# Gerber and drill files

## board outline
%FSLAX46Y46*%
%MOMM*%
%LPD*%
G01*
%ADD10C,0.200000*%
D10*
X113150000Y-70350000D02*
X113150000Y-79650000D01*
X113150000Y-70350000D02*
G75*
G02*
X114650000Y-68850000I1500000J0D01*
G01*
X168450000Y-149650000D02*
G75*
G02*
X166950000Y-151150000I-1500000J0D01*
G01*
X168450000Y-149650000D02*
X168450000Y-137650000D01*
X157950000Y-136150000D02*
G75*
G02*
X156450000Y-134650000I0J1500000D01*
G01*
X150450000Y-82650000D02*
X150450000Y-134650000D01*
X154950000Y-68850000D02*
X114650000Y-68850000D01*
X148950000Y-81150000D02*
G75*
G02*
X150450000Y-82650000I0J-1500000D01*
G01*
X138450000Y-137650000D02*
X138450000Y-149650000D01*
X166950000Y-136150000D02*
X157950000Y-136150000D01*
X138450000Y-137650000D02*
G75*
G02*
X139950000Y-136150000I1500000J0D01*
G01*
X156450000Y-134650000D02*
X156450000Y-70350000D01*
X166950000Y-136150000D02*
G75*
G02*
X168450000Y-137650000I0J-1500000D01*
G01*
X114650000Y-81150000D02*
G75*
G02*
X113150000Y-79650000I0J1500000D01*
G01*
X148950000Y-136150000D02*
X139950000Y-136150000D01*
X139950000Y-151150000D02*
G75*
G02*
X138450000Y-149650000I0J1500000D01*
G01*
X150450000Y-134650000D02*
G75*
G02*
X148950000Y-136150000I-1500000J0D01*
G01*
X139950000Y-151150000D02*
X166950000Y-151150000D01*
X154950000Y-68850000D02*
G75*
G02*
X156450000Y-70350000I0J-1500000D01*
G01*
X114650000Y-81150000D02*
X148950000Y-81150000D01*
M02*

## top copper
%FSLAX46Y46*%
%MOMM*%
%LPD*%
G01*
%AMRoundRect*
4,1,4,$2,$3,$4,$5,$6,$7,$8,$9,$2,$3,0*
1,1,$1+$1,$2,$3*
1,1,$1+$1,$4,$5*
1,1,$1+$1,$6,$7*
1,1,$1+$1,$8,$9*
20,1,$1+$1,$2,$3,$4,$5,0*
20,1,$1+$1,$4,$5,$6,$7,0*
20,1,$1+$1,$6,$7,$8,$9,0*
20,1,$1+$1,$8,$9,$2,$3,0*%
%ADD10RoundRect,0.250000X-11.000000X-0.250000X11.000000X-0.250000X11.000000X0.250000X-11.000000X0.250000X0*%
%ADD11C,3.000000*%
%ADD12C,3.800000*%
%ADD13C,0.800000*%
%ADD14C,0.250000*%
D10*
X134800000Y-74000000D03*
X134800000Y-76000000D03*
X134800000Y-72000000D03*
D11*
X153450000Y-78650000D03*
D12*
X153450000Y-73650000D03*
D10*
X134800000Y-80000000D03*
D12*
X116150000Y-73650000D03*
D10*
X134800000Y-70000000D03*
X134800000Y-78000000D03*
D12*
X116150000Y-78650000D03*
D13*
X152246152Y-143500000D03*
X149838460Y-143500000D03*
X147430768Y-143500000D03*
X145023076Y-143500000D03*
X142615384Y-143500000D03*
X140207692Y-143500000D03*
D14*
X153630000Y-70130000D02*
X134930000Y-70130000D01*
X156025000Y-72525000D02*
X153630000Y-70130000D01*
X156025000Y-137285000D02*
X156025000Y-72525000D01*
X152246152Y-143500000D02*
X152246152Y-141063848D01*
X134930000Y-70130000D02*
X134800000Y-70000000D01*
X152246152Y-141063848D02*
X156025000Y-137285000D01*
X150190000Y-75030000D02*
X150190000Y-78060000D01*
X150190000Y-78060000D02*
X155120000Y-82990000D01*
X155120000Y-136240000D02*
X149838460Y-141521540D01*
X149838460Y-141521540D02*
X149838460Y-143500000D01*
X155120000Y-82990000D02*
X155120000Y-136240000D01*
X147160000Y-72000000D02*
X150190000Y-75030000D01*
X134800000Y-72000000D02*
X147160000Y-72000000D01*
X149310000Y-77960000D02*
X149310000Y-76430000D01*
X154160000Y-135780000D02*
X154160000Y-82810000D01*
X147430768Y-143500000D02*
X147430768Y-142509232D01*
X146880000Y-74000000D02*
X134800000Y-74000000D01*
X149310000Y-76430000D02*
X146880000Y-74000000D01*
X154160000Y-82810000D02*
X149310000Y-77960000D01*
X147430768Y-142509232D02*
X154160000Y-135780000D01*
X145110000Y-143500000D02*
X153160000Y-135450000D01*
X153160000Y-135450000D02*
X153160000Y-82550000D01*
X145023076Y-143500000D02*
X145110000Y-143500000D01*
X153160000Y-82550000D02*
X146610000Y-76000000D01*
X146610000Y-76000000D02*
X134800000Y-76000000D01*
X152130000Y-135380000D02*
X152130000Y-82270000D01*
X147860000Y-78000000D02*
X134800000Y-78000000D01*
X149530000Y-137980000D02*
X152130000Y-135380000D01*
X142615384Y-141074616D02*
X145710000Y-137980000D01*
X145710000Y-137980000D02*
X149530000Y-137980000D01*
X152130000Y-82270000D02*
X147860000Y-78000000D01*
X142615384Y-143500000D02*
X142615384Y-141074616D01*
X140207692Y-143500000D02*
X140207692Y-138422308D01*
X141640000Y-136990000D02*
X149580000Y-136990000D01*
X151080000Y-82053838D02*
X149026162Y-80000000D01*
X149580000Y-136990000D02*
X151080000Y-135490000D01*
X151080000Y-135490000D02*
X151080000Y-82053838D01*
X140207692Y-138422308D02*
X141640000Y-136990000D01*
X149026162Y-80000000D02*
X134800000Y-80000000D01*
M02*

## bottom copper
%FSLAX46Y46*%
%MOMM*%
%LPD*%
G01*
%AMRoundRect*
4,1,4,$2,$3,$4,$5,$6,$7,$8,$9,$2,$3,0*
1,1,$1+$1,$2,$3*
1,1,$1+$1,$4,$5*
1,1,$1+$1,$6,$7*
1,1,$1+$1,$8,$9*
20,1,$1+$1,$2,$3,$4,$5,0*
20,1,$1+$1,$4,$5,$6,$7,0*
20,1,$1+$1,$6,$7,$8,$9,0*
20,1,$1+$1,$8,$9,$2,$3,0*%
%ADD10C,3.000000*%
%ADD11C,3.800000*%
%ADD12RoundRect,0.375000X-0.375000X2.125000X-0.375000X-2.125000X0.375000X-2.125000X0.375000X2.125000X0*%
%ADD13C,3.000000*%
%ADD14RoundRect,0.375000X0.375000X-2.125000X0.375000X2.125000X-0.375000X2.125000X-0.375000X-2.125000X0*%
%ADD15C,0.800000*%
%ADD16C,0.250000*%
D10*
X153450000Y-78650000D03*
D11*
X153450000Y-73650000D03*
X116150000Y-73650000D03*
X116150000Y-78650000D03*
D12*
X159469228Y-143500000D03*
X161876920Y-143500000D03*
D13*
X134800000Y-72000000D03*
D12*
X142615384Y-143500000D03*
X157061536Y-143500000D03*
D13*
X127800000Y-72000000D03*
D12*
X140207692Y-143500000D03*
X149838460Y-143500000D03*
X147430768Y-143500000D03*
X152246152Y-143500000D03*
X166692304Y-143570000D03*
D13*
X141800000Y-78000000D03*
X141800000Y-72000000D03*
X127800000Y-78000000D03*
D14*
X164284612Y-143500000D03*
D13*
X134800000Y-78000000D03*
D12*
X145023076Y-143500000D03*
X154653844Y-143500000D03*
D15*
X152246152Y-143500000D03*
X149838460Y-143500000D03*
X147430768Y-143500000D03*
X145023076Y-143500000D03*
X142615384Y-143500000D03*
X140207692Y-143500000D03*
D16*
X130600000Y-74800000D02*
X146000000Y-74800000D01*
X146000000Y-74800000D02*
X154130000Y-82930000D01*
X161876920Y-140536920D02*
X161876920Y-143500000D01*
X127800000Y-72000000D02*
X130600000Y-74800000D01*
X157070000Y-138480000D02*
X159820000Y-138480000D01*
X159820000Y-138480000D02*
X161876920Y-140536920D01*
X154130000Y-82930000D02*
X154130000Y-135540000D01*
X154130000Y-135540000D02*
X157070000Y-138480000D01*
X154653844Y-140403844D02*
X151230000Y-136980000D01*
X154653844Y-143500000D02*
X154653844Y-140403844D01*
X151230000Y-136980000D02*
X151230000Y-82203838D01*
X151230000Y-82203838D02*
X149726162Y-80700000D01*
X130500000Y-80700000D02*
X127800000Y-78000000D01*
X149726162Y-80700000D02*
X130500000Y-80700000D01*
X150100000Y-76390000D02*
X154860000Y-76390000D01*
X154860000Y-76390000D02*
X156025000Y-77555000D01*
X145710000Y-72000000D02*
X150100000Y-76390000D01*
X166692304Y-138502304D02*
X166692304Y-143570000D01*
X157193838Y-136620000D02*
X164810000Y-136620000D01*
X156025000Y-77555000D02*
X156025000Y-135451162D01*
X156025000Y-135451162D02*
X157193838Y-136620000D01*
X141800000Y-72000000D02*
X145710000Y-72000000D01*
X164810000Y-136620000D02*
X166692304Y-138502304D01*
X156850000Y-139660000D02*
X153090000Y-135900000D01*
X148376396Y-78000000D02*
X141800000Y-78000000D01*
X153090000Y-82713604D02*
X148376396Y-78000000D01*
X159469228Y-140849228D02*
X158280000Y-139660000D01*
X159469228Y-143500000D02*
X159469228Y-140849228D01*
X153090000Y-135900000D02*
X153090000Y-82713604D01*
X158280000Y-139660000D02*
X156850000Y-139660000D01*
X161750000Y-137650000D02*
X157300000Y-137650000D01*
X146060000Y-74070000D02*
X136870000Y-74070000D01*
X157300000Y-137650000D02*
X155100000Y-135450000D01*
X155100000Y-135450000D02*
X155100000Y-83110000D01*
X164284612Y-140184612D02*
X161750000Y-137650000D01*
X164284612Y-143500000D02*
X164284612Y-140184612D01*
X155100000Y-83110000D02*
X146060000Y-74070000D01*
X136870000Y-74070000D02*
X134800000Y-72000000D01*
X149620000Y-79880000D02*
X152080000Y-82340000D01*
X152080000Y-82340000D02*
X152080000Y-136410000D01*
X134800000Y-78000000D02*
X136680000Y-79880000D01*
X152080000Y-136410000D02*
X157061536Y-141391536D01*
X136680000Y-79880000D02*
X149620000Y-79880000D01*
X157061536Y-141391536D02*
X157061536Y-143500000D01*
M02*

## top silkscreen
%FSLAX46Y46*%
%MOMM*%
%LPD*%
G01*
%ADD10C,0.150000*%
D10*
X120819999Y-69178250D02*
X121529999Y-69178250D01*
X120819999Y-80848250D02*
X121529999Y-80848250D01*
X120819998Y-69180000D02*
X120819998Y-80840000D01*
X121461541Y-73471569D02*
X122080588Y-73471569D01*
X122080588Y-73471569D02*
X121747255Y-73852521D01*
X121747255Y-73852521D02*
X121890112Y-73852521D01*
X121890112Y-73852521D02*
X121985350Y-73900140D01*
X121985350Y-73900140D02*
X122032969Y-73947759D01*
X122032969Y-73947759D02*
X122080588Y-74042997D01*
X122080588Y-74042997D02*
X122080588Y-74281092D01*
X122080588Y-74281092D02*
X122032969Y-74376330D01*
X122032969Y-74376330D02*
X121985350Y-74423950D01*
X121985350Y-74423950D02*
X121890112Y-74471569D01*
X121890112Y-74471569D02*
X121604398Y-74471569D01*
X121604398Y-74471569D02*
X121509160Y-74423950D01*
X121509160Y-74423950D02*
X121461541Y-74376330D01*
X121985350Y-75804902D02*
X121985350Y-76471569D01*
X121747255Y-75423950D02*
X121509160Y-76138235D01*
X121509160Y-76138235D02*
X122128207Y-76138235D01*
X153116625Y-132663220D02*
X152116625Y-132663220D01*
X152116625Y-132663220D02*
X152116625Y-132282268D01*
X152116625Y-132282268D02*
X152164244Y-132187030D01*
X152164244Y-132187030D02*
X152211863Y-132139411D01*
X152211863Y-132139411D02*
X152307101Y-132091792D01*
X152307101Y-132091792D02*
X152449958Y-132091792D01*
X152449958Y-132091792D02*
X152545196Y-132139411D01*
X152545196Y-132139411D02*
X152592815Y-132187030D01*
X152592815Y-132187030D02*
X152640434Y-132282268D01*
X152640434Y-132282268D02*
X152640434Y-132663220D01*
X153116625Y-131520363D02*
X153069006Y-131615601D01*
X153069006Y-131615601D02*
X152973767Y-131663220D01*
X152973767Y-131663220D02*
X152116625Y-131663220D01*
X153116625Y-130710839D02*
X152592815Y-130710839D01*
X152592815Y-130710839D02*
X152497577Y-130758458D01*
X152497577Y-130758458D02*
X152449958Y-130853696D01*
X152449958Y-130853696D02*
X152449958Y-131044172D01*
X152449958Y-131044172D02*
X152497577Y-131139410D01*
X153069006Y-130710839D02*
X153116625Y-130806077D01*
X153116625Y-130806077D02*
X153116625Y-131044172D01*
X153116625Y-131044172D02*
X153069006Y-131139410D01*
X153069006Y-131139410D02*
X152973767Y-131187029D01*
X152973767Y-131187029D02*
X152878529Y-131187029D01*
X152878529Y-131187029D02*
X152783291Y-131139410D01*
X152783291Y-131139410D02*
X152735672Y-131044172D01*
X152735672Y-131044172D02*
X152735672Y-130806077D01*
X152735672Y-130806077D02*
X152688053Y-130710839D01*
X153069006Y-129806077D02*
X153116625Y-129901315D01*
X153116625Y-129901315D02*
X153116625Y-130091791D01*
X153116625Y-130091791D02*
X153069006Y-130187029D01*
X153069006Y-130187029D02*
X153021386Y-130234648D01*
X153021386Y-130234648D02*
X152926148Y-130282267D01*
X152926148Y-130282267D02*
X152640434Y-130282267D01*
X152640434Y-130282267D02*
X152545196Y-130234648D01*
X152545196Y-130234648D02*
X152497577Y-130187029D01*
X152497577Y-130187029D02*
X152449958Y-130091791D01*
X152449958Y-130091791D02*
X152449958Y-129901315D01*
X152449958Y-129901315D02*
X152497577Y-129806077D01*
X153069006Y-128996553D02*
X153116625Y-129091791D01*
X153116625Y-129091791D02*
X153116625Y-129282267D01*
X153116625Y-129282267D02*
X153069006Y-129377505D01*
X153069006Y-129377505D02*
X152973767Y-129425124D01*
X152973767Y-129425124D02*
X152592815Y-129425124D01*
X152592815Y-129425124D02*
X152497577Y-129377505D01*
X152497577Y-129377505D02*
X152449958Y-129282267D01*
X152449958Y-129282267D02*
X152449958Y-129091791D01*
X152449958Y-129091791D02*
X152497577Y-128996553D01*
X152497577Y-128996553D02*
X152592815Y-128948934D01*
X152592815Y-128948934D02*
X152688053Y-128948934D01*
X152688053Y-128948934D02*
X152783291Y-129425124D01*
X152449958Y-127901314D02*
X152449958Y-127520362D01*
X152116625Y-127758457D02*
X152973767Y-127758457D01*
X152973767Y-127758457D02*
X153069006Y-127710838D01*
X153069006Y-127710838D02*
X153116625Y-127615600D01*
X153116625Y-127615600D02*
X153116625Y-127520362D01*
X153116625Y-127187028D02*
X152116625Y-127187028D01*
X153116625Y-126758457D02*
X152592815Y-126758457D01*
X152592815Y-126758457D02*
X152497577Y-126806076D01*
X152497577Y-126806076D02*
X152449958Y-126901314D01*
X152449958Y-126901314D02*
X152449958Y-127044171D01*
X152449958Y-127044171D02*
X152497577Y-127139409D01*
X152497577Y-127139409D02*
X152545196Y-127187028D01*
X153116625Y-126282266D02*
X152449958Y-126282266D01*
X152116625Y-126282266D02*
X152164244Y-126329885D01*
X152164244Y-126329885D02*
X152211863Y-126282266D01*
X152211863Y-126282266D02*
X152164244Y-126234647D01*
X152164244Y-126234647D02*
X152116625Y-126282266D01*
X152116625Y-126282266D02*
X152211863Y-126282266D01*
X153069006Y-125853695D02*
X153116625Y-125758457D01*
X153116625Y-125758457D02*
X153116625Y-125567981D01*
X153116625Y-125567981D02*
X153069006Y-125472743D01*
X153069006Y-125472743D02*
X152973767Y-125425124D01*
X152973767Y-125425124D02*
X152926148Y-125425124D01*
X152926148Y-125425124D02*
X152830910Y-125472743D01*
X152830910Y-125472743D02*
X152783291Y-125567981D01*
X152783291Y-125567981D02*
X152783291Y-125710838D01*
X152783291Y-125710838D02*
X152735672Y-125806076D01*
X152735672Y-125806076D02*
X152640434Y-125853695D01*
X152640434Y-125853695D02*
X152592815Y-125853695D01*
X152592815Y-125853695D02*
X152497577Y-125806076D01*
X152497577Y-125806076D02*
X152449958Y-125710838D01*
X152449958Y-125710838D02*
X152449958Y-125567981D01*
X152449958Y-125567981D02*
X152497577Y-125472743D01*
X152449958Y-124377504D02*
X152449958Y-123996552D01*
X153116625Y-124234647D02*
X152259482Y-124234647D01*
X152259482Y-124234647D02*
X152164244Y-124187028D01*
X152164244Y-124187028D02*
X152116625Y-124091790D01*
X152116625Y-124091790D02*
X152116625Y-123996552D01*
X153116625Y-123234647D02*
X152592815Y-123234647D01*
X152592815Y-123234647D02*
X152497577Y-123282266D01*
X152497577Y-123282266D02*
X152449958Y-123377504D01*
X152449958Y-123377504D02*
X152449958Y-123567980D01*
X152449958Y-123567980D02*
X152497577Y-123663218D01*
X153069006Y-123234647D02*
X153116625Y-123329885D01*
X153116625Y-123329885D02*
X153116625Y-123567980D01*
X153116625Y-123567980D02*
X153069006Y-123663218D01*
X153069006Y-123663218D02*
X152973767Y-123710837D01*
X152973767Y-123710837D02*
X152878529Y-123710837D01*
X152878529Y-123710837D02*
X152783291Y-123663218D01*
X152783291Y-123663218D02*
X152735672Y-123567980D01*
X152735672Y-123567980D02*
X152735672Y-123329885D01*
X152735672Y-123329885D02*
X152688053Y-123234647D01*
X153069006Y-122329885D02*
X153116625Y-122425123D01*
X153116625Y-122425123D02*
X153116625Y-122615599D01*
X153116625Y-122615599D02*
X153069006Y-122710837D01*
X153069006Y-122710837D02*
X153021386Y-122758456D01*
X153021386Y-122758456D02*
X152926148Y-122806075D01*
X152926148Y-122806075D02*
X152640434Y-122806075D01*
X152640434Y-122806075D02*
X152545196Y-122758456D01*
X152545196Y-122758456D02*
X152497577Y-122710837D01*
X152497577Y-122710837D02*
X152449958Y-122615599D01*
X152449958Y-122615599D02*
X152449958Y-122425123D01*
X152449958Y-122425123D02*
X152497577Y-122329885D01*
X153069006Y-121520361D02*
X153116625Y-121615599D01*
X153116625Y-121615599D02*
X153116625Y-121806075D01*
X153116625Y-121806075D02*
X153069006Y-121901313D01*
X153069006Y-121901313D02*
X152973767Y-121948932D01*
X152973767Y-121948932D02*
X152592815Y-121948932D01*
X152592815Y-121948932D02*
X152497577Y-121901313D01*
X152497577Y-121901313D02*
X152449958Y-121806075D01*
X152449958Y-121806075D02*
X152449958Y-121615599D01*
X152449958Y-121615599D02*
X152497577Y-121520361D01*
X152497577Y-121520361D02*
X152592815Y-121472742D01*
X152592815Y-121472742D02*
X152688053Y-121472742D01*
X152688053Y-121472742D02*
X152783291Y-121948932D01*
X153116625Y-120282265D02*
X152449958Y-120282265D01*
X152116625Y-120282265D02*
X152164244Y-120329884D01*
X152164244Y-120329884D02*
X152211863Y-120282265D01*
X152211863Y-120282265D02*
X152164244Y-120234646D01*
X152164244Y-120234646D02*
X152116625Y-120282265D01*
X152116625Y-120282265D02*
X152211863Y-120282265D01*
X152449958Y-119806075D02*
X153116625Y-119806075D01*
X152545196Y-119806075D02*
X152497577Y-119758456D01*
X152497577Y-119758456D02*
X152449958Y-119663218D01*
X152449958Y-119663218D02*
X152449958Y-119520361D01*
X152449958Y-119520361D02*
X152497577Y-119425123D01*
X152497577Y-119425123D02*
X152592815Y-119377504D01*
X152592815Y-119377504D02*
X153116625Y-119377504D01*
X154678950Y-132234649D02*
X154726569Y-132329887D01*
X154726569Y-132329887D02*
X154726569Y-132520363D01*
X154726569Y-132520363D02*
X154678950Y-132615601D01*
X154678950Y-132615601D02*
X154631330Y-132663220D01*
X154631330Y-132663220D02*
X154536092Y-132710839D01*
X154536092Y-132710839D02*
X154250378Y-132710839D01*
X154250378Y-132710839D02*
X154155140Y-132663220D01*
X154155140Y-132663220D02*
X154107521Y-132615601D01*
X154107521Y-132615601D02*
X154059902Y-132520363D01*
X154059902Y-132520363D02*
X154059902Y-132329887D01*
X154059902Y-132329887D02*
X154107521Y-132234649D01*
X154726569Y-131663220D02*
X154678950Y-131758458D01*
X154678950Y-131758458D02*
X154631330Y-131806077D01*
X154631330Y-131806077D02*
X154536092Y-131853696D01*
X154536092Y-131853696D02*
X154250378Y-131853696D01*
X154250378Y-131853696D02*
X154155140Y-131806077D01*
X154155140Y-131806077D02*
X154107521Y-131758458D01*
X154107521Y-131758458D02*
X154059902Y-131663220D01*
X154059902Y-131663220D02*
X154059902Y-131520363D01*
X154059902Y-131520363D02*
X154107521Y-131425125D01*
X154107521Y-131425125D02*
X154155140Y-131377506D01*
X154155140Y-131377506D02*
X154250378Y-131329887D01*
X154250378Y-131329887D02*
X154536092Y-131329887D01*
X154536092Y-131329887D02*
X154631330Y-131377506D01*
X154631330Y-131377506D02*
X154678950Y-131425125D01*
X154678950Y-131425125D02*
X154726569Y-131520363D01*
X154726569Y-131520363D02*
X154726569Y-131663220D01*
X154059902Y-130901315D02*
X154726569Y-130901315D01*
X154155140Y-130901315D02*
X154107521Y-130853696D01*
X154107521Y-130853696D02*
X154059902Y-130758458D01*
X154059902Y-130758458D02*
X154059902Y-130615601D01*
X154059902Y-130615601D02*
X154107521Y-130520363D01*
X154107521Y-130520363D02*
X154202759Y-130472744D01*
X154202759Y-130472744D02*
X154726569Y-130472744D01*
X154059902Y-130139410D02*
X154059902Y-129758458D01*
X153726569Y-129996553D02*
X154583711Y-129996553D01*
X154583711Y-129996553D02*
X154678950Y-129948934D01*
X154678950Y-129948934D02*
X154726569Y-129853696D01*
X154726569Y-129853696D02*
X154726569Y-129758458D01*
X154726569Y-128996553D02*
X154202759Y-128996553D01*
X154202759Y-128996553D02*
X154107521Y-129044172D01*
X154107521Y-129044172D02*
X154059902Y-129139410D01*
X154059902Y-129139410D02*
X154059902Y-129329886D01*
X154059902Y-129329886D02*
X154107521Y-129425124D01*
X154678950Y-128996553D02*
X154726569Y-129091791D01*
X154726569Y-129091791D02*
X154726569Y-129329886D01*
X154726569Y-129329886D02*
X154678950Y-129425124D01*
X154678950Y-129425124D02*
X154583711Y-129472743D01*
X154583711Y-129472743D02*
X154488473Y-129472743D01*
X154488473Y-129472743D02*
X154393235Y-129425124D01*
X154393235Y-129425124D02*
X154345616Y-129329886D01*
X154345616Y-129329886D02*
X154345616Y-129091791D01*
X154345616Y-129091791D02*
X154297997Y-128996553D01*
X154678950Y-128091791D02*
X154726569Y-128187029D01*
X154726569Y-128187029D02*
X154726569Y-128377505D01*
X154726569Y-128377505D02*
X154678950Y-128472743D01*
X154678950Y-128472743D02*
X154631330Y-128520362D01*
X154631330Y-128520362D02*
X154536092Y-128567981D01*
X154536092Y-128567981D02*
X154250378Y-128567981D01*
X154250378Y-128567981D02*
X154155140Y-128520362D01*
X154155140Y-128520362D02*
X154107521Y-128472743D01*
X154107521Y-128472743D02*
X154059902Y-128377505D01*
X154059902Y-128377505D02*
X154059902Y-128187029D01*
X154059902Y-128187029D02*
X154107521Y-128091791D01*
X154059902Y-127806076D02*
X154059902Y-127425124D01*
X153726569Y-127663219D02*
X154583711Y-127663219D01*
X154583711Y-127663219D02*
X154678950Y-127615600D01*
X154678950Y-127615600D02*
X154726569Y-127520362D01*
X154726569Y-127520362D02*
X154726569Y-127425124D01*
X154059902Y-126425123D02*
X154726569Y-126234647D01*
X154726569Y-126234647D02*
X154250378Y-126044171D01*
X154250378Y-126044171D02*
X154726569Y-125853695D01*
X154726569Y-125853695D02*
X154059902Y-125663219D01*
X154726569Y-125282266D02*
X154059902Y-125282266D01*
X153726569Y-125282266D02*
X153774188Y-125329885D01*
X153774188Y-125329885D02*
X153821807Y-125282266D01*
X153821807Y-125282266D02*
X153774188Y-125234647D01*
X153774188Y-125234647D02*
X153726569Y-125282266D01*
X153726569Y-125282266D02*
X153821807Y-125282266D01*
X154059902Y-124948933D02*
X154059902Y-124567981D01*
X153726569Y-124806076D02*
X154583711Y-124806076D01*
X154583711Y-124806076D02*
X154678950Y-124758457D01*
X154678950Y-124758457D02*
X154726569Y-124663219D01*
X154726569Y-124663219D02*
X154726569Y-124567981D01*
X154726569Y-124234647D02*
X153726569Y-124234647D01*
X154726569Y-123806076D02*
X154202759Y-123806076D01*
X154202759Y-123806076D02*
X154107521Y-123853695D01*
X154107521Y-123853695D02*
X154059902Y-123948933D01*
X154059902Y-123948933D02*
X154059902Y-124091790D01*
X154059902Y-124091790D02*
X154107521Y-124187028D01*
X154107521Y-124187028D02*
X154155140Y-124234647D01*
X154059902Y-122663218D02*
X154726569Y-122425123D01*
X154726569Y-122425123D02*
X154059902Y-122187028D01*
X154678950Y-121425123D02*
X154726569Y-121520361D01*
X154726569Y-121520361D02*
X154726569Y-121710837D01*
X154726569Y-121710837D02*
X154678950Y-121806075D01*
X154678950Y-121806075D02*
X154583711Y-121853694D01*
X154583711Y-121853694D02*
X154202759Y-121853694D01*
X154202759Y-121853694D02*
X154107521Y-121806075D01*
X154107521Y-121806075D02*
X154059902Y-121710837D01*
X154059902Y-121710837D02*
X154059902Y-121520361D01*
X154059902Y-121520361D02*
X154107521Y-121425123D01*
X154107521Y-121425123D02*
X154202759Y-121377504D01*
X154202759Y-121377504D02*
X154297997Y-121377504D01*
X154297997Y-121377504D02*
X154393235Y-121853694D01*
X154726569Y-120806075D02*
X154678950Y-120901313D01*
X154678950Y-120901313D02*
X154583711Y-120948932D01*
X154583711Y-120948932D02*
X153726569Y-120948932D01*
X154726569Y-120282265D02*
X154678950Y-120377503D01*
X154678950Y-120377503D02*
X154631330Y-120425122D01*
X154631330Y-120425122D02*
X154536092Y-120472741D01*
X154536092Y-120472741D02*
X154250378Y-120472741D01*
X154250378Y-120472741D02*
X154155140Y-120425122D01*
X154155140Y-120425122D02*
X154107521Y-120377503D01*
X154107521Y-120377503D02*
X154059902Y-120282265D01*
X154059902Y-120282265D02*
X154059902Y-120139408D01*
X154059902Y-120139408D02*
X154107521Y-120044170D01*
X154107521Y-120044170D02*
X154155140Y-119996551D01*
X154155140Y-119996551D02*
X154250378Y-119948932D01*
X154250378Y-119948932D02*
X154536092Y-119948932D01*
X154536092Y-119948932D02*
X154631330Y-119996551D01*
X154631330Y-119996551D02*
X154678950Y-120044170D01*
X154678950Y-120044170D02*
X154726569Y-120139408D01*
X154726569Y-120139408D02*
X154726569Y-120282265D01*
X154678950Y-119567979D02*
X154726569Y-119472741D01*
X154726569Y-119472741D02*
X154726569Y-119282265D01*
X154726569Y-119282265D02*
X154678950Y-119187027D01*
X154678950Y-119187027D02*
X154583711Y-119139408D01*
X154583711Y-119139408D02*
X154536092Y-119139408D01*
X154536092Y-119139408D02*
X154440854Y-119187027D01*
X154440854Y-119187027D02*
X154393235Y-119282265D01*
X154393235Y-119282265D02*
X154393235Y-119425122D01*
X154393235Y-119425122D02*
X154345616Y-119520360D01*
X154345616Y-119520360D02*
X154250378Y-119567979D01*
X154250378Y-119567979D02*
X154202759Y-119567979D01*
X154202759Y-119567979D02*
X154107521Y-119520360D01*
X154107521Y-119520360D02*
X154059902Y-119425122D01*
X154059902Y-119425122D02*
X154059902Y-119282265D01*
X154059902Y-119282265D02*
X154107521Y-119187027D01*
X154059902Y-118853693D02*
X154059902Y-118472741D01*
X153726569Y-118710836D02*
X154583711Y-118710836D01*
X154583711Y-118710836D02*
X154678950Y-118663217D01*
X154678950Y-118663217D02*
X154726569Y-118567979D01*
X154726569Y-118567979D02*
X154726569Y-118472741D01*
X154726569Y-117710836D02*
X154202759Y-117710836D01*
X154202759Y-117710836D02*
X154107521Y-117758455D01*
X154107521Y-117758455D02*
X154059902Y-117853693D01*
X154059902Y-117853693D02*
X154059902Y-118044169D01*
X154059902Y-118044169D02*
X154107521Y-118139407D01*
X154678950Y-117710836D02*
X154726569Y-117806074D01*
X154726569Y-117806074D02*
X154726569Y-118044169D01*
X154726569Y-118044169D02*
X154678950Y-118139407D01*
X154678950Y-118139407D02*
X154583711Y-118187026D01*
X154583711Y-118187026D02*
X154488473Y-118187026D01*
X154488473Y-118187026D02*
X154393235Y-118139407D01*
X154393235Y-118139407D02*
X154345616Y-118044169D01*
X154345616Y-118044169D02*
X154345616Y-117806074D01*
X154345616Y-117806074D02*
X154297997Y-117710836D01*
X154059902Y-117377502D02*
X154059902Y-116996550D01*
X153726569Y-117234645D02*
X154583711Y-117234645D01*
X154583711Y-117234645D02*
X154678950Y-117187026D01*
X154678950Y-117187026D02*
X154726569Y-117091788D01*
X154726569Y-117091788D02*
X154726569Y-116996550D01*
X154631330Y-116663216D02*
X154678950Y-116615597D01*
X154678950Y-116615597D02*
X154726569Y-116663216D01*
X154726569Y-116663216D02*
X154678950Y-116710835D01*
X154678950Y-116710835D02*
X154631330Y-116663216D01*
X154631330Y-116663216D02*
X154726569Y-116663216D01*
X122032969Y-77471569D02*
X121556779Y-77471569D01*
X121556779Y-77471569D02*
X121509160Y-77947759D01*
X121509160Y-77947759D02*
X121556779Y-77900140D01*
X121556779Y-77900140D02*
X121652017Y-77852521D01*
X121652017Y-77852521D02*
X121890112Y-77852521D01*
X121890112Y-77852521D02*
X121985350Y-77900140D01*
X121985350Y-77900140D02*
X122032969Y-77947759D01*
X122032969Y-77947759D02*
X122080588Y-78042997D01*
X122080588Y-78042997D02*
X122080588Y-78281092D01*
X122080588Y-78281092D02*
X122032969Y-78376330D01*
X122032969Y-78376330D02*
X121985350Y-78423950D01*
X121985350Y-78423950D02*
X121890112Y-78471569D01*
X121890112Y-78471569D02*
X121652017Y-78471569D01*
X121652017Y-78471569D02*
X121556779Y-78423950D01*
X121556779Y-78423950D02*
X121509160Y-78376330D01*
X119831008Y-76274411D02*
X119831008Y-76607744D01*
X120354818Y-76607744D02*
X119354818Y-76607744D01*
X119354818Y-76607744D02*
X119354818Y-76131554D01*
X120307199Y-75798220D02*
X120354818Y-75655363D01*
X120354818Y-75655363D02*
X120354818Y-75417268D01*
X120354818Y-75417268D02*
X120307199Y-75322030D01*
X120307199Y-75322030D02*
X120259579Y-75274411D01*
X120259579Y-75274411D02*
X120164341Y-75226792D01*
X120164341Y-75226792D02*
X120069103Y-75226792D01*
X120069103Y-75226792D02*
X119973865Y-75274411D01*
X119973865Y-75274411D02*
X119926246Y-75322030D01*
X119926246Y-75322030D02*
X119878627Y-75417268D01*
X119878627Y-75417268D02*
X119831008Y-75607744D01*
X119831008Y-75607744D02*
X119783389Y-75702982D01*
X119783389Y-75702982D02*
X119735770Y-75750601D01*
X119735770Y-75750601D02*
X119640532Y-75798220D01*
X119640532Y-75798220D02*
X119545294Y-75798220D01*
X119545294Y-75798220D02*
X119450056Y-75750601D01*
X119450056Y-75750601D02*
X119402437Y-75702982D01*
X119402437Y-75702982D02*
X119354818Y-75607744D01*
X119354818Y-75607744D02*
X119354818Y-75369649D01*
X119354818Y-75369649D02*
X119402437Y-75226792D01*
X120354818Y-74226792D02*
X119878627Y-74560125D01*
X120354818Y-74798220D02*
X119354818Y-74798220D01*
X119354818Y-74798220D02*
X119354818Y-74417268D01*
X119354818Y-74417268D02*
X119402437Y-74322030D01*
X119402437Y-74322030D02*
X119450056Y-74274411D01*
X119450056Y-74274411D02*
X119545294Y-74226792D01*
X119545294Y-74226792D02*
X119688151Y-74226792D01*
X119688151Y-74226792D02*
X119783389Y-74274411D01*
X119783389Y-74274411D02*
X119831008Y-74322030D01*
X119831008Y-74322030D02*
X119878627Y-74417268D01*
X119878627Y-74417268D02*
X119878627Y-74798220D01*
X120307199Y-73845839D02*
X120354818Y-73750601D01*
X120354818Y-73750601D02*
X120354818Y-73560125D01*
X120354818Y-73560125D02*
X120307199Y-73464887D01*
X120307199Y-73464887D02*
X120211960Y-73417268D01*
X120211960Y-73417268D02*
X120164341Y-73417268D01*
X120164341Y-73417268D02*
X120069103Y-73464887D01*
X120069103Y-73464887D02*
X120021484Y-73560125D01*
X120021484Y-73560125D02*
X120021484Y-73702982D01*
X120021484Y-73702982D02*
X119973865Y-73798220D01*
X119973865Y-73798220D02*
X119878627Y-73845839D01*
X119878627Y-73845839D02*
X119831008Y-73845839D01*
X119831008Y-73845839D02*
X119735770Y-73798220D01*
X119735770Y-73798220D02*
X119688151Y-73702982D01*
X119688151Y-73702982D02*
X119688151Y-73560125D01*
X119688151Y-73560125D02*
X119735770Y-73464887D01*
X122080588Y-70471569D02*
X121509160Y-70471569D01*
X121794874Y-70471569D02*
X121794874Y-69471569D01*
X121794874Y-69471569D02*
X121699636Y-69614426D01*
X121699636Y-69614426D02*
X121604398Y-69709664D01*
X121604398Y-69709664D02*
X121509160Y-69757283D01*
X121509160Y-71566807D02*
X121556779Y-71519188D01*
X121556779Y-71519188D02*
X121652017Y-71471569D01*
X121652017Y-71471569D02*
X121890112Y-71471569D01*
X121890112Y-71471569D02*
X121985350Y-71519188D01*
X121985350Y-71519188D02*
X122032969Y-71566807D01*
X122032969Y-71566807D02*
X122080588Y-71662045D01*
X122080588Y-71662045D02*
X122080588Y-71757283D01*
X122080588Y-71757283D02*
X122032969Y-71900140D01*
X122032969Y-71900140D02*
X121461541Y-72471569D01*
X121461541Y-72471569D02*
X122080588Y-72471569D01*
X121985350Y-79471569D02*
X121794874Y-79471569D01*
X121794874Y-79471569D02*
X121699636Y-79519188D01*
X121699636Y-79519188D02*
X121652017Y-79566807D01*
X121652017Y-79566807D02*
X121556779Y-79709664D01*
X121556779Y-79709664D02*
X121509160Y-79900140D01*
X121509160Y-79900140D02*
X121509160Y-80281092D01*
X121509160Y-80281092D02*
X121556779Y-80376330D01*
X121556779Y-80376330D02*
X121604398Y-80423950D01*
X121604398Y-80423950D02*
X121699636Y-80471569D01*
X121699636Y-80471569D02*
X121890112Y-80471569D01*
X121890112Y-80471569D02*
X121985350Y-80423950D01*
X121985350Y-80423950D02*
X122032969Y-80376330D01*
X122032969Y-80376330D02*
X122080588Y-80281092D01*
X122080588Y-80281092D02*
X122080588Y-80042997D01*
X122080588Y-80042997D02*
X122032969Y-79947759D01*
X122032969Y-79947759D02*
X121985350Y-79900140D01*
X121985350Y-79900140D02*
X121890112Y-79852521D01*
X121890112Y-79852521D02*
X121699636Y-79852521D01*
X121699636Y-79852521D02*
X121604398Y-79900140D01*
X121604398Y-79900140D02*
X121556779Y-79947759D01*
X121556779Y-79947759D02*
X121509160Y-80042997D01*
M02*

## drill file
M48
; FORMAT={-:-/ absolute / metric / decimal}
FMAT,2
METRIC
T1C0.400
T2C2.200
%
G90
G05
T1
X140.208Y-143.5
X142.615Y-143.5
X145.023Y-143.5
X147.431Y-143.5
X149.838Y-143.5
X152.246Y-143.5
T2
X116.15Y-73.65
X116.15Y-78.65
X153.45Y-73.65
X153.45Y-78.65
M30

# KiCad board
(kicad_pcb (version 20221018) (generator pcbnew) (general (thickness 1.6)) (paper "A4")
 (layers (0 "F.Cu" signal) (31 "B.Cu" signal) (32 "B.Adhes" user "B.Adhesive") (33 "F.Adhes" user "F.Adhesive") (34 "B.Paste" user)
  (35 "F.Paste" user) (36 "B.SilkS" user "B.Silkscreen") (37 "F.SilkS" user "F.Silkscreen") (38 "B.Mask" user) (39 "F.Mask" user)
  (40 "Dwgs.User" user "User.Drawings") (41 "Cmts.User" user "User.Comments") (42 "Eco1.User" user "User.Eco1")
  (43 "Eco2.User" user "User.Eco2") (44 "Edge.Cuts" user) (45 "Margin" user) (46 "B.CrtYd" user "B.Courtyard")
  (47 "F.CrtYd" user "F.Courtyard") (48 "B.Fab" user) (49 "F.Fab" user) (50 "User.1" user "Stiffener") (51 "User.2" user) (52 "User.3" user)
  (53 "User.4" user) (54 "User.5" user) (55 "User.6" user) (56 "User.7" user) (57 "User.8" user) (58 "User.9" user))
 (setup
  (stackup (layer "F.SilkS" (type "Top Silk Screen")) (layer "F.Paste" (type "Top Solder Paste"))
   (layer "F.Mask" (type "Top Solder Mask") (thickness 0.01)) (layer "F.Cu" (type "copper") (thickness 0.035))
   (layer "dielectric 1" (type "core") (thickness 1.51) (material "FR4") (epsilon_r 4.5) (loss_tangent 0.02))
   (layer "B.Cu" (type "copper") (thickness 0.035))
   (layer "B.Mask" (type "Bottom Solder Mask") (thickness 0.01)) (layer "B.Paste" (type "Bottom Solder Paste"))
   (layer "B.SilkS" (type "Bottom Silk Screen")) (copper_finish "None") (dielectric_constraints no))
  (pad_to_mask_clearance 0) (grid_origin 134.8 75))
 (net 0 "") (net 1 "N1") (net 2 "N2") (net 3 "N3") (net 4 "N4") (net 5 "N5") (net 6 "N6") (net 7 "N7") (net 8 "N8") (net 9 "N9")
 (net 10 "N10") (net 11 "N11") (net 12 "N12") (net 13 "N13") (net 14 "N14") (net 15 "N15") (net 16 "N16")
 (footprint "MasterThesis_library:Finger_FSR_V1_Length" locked (layer "F.Cu") (at 134.8 74)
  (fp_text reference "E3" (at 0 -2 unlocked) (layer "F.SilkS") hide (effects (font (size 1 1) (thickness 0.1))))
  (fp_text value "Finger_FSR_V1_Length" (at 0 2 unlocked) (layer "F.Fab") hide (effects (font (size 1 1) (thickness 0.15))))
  (pad "1" smd roundrect locked (at 0 0) (size 22.5 1) (layers "F.Cu" "F.Paste" "F.Mask") (roundrect_rratio 0.25) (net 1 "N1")
   (thermal_bridge_angle 45)))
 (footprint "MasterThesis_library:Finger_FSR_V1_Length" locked (layer "F.Cu") (at 134.8 76)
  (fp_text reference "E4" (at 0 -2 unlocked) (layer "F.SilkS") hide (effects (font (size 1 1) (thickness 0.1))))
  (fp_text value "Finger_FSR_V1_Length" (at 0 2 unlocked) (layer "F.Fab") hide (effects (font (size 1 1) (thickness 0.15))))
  (pad "1" smd roundrect locked (at 0 0) (size 22.5 1) (layers "F.Cu" "F.Paste" "F.Mask") (roundrect_rratio 0.25) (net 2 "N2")
   (thermal_bridge_angle 45)))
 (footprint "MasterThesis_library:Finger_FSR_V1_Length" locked (layer "F.Cu") (at 134.8 72)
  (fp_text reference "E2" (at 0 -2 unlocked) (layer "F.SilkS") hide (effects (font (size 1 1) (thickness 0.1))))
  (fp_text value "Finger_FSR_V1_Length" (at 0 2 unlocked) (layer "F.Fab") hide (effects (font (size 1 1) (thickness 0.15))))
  (pad "1" smd roundrect locked (at 0 0) (size 22.5 1) (layers "F.Cu" "F.Paste" "F.Mask") (roundrect_rratio 0.25) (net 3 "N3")
   (thermal_bridge_angle 45)))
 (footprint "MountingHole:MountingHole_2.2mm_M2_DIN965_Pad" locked (layer "F.Cu") (at 153.45 78.65)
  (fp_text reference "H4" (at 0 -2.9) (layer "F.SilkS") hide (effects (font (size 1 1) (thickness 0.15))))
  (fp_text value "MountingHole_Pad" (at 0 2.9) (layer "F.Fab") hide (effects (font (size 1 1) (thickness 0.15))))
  (pad "1" thru_hole circle locked (at 0 0) (size 3 3) (drill 2.2) (layers "*.Cu" "*.Mask") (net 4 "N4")))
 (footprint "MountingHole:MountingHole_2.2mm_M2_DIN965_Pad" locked (layer "F.Cu") (at 153.45 73.65)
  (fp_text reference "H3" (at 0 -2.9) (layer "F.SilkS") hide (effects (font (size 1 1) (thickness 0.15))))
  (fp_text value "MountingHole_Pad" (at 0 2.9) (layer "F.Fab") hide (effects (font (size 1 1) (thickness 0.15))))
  (pad "1" thru_hole circle locked (at 0 0) (size 3.8 3.8) (drill 2.2) (layers "*.Cu" "*.Mask") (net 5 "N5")))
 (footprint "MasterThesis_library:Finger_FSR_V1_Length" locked (layer "F.Cu") (at 134.8 80)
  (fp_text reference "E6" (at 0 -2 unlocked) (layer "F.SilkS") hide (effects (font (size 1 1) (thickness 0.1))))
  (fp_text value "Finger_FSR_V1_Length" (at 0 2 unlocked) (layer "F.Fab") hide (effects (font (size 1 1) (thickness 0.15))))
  (pad "1" smd roundrect locked (at 0 0) (size 22.5 1) (layers "F.Cu" "F.Paste" "F.Mask") (roundrect_rratio 0.25) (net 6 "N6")
   (thermal_bridge_angle 45)))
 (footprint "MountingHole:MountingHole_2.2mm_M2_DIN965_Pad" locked (layer "F.Cu") (at 116.15 73.65)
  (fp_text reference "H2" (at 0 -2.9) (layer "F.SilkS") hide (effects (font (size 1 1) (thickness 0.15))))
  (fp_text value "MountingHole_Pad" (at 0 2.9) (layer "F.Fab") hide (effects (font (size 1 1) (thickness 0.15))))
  (pad "1" thru_hole circle locked (at 0 0) (size 3.8 3.8) (drill 2.2) (layers "*.Cu" "*.Mask") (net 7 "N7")))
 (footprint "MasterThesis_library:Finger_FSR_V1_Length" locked (layer "F.Cu") (at 134.8 70)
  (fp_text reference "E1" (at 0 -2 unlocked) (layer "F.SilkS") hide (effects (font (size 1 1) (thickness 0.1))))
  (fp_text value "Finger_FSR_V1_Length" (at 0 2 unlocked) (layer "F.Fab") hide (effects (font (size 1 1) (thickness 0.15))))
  (pad "1" smd roundrect locked (at 0 0) (size 22.5 1) (layers "F.Cu" "F.Paste" "F.Mask") (roundrect_rratio 0.25) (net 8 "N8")
   (thermal_bridge_angle 45)))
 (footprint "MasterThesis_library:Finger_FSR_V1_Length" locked (layer "F.Cu") (at 134.8 78)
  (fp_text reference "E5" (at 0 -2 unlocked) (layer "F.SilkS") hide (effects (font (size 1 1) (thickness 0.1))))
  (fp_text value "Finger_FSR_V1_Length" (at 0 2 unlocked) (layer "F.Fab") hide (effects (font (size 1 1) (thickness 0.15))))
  (pad "1" smd roundrect locked (at 0 0) (size 22.5 1) (layers "F.Cu" "F.Paste" "F.Mask") (roundrect_rratio 0.25) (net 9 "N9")
   (thermal_bridge_angle 45)))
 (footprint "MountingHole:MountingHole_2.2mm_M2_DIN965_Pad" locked (layer "F.Cu") (at 116.15 78.65)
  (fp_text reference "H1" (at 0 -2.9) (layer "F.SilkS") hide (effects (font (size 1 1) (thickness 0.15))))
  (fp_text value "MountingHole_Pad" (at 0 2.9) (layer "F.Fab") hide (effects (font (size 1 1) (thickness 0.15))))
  (pad "1" thru_hole circle locked (at 0 0) (size 3.8 3.8) (drill 2.2) (layers "*.Cu" "*.Mask") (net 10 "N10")))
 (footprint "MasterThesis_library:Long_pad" (layer "B.Cu") (at 159.469228 143.5 -90)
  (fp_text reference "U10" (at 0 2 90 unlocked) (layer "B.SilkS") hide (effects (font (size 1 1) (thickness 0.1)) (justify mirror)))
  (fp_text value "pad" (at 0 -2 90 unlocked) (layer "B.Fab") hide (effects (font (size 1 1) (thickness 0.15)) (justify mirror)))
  (pad "1" smd roundrect (at 0 0 270) (size 5 1.5) (layers "B.Cu" "B.Paste" "B.Mask") (roundrect_rratio 0.25) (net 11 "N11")
   (thermal_bridge_angle 45)))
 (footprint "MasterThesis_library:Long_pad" (layer "B.Cu") (at 161.87692 143.5 -90)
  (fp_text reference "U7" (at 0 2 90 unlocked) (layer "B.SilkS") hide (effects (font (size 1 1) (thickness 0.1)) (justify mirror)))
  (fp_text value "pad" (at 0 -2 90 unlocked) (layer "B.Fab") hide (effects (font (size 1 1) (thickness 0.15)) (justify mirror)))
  (pad "1" smd roundrect (at 0 0 270) (size 5 1.5) (layers "B.Cu" "B.Paste" "B.Mask") (roundrect_rratio 0.25) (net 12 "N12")
   (thermal_bridge_angle 45)))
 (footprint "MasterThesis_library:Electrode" (layer "B.Cu") (at 134.8 72 180)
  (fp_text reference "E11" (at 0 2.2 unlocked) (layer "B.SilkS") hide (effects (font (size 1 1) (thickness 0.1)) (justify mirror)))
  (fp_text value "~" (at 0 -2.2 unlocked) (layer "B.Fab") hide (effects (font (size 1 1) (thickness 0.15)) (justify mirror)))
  (pad "1" smd circle (at 0 0 180) (size 3 3) (layers "B.Cu" "B.Paste" "B.Mask") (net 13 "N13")))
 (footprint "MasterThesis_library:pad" (layer "B.Cu") (at 142.615384 143.5 -90)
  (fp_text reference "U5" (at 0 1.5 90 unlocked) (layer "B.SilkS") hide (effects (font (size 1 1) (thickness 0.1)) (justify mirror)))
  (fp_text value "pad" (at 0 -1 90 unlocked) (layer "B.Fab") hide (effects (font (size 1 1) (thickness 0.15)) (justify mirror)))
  (pad "1" smd roundrect (at 0 0 270) (size 5 1.5) (layers "B.Cu" "B.Paste" "B.Mask") (roundrect_rratio 0.25) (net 9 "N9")
   (thermal_bridge_angle 45)))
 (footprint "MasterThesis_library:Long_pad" (layer "B.Cu") (at 157.061536 143.5 -90)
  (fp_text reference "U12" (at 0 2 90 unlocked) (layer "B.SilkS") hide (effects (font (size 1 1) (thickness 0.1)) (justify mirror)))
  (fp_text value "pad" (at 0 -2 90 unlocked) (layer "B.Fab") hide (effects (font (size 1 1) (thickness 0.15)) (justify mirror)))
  (pad "1" smd roundrect (at 0 0 270) (size 5 1.5) (layers "B.Cu" "B.Paste" "B.Mask") (roundrect_rratio 0.25) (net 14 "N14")
   (thermal_bridge_angle 45)))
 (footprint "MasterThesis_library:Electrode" (layer "B.Cu") (at 127.8 72 180)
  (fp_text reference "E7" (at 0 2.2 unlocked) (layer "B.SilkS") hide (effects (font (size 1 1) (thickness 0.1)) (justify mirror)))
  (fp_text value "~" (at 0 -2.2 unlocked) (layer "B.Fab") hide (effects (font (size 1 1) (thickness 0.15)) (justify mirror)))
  (pad "1" smd circle (at 0 0 180) (size 3 3) (layers "B.Cu" "B.Paste" "B.Mask") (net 12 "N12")))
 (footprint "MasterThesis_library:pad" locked (layer "B.Cu") (at 140.207692 143.5 -90)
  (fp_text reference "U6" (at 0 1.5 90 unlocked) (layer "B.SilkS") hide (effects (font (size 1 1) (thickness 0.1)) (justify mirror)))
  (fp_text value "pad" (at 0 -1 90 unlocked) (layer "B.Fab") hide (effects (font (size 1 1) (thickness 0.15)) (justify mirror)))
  (pad "1" smd roundrect locked (at 0 0 270) (size 5 1.5) (layers "B.Cu" "B.Paste" "B.Mask") (roundrect_rratio 0.25) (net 6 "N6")
   (thermal_bridge_angle 45)))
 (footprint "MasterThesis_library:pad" (layer "B.Cu") (at 149.83846 143.5 -90)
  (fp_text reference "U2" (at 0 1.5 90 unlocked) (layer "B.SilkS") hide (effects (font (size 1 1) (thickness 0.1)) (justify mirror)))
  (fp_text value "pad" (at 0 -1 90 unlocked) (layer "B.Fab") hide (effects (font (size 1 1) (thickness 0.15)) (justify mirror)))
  (pad "1" smd roundrect (at 0 0 270) (size 5 1.5) (layers "B.Cu" "B.Paste" "B.Mask") (roundrect_rratio 0.25) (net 3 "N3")
   (thermal_bridge_angle 45)))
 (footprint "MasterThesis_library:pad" (layer "B.Cu") (at 147.430768 143.5 -90)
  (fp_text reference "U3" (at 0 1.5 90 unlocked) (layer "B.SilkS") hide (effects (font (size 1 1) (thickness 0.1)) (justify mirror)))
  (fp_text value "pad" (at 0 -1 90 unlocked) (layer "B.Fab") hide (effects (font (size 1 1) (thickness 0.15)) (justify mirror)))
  (pad "1" smd roundrect (at 0 0 270) (size 5 1.5) (layers "B.Cu" "B.Paste" "B.Mask") (roundrect_rratio 0.25) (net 1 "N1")
   (thermal_bridge_angle 45)))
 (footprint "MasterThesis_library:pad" (layer "B.Cu") (at 152.246152 143.5 -90)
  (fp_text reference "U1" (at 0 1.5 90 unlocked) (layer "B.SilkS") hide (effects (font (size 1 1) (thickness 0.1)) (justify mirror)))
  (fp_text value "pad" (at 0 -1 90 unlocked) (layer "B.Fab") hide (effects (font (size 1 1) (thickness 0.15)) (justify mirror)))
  (pad "1" smd roundrect (at 0 0 270) (size 5 1.5) (layers "B.Cu" "B.Paste" "B.Mask") (roundrect_rratio 0.25) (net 8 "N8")
   (thermal_bridge_angle 45)))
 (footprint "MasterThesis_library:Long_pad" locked (layer "B.Cu") (at 166.692304 143.57 -90)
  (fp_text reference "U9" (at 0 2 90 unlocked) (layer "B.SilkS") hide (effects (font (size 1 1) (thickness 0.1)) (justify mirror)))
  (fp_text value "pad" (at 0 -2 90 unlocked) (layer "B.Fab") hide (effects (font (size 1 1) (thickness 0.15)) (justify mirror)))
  (pad "1" smd roundrect locked (at 0 0 270) (size 5 1.5) (layers "B.Cu" "B.Paste" "B.Mask") (roundrect_rratio 0.25) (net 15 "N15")
   (thermal_bridge_angle 45)))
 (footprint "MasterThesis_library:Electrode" (layer "B.Cu") (at 141.8 78 180)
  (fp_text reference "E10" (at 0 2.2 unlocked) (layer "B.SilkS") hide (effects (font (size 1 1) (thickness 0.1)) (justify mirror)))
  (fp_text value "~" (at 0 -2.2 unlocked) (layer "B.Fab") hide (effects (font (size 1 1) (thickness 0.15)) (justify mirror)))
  (pad "1" smd circle (at 0 0 180) (size 3 3) (layers "B.Cu" "B.Paste" "B.Mask") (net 11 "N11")))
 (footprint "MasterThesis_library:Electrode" (layer "B.Cu") (at 141.8 72 180)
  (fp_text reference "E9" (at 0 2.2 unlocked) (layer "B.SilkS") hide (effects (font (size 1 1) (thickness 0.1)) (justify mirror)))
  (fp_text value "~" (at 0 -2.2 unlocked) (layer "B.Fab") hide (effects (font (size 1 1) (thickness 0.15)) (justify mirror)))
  (pad "1" smd circle (at 0 0 180) (size 3 3) (layers "B.Cu" "B.Paste" "B.Mask") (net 15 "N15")))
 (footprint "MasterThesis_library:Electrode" (layer "B.Cu") (at 127.8 78 180)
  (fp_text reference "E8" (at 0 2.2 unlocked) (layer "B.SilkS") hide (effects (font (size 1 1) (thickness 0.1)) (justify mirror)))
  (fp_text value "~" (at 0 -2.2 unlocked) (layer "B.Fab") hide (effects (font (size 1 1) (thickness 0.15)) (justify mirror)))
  (pad "1" smd circle (at 0 0 180) (size 3 3) (layers "B.Cu" "B.Paste" "B.Mask") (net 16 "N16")))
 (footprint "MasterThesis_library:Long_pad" (layer "B.Cu") (at 164.284612 143.5 90)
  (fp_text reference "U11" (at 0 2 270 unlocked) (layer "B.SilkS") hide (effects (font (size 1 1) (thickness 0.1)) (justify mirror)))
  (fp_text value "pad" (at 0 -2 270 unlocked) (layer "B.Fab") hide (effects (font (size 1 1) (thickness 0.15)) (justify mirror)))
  (pad "1" smd roundrect (at 0 0 90) (size 5 1.5) (layers "B.Cu" "B.Paste" "B.Mask") (roundrect_rratio 0.25) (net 13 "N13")
   (thermal_bridge_angle 45)))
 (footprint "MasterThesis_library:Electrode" (layer "B.Cu") (at 134.8 78 180)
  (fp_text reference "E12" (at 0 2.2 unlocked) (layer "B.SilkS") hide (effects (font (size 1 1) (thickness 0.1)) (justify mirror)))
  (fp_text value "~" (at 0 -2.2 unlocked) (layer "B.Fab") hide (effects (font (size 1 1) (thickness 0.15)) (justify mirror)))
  (pad "1" smd circle (at 0 0 180) (size 3 3) (layers "B.Cu" "B.Paste" "B.Mask") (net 14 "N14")))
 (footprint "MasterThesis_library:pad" (layer "B.Cu") (at 145.023076 143.5 -90)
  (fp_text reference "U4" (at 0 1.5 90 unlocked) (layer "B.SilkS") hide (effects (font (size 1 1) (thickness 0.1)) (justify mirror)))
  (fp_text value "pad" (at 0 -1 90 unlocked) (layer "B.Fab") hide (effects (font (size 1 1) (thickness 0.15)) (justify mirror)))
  (pad "1" smd roundrect (at 0 0 270) (size 5 1.5) (layers "B.Cu" "B.Paste" "B.Mask") (roundrect_rratio 0.25) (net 2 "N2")
   (thermal_bridge_angle 45)))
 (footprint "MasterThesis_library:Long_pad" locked (layer "B.Cu") (at 154.653844 143.5 -90)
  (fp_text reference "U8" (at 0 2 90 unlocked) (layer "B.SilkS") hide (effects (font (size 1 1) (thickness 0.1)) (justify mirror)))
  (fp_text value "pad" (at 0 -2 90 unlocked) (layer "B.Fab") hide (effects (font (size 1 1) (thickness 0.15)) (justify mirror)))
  (pad "1" smd roundrect locked (at 0 0 270) (size 5 1.5) (layers "B.Cu" "B.Paste" "B.Mask") (roundrect_rratio 0.25) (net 16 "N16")
   (thermal_bridge_angle 45)))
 (gr_line (start 120.819999 69.17825) (end 121.529999 69.17825) (stroke (width 0.15) (type default)) (layer "F.SilkS"))
 (gr_line (start 120.819999 80.84825) (end 121.529999 80.84825) (stroke (width 0.15) (type default)) (layer "F.SilkS"))
 (gr_line (start 120.819998 69.18) (end 120.819998 80.84) (stroke (width 0.15) (type default)) (layer "F.SilkS"))
 (gr_line locked (start 113.15 70.35) (end 113.15 79.65) (stroke (width 0.2) (type solid)) (layer "Edge.Cuts"))
 (gr_arc locked (start 113.15 70.35) (mid 113.58934 69.28934) (end 114.65 68.85) (stroke (width 0.2) (type solid)) (layer "Edge.Cuts"))
 (gr_arc locked (start 168.45 149.65) (mid 168.01066 150.71066) (end 166.95 151.15) (stroke (width 0.2) (type solid)) (layer "Edge.Cuts"))
 (gr_line locked (start 168.45 149.65) (end 168.45 137.65) (stroke (width 0.2) (type solid)) (layer "Edge.Cuts"))
 (gr_arc locked (start 157.95 136.15) (mid 156.88934 135.71066) (end 156.45 134.65) (stroke (width 0.2) (type solid)) (layer "Edge.Cuts"))
 (gr_line locked (start 150.45 82.65) (end 150.45 134.65) (stroke (width 0.2) (type solid)) (layer "Edge.Cuts"))
 (gr_line locked (start 154.95 68.85) (end 114.65 68.85) (stroke (width 0.2) (type solid)) (layer "Edge.Cuts"))
 (gr_arc locked (start 148.95 81.15) (mid 150.01066 81.58934) (end 150.45 82.65) (stroke (width 0.2) (type solid)) (layer "Edge.Cuts"))
 (gr_line locked (start 138.45 137.65) (end 138.45 149.65) (stroke (width 0.2) (type solid)) (layer "Edge.Cuts"))
 (gr_line locked (start 166.95 136.15) (end 157.95 136.15) (stroke (width 0.2) (type solid)) (layer "Edge.Cuts"))
 (gr_arc locked (start 138.45 137.65) (mid 138.88934 136.58934) (end 139.95 136.15) (stroke (width 0.2) (type solid)) (layer "Edge.Cuts"))
 (gr_line locked (start 156.45 134.65) (end 156.45 70.35) (stroke (width 0.2) (type solid)) (layer "Edge.Cuts"))
 (gr_arc locked (start 166.95 136.15) (mid 168.01066 136.58934) (end 168.45 137.65) (stroke (width 0.2) (type solid)) (layer "Edge.Cuts"))
 (gr_arc locked (start 114.65 81.15) (mid 113.58934 80.71066) (end 113.15 79.65) (stroke (width 0.2) (type solid)) (layer "Edge.Cuts"))
 (gr_line locked (start 148.95 136.15) (end 139.95 136.15) (stroke (width 0.2) (type solid)) (layer "Edge.Cuts"))
 (gr_arc locked (start 139.95 151.15) (mid 138.88934 150.71066) (end 138.45 149.65) (stroke (width 0.2) (type solid)) (layer "Edge.Cuts"))
 (gr_arc locked (start 150.45 134.65) (mid 150.01066 135.71066) (end 148.95 136.15) (stroke (width 0.2) (type solid)) (layer "Edge.Cuts"))
 (gr_line locked (start 139.95 151.15) (end 166.95 151.15) (stroke (width 0.2) (type solid)) (layer "Edge.Cuts"))
 (gr_arc locked (start 154.95 68.85) (mid 156.01066 69.28934) (end 156.45 70.35) (stroke (width 0.2) (type solid)) (layer "Edge.Cuts"))
 (gr_line locked (start 114.65 81.15) (end 148.95 81.15) (stroke (width 0.2) (type solid)) (layer "Edge.Cuts"))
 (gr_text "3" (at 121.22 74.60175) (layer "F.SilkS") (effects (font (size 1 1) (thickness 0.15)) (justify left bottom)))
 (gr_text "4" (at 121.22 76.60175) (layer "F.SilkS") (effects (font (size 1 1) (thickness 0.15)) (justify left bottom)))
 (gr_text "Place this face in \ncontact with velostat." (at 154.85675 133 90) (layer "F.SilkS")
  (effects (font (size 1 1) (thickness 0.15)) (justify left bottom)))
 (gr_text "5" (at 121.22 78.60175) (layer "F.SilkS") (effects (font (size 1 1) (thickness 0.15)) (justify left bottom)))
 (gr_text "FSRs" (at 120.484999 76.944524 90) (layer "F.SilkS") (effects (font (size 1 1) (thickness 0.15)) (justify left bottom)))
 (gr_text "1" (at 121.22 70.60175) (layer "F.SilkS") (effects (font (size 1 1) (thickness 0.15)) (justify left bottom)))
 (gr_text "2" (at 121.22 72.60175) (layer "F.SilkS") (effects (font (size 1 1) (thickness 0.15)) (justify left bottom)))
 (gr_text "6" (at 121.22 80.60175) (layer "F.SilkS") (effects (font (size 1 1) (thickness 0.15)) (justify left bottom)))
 (segment (start 153.63 70.13) (end 134.93 70.13) (width 0.25) (layer "F.Cu") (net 8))
 (segment (start 156.025 72.525) (end 153.63 70.13) (width 0.25) (layer "F.Cu") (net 8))
 (segment (start 156.025 137.285) (end 156.025 72.525) (width 0.25) (layer "F.Cu") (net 8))
 (segment (start 152.246152 143.5) (end 152.246152 141.063848) (width 0.25) (layer "F.Cu") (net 8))
 (segment (start 134.93 70.13) (end 134.8 70) (width 0.25) (layer "F.Cu") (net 8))
 (segment (start 152.246152 141.063848) (end 156.025 137.285) (width 0.25) (layer "F.Cu") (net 8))
 (via (at 152.246152 143.5) (size 0.8) (drill 0.4) (layers "F.Cu" "B.Cu") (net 8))
 (segment (start 150.19 75.03) (end 150.19 78.06) (width 0.25) (layer "F.Cu") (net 3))
 (segment (start 150.19 78.06) (end 155.12 82.99) (width 0.25) (layer "F.Cu") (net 3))
 (segment (start 155.12 136.24) (end 149.83846 141.52154) (width 0.25) (layer "F.Cu") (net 3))
 (segment (start 149.83846 141.52154) (end 149.83846 143.5) (width 0.25) (layer "F.Cu") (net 3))
 (segment (start 155.12 82.99) (end 155.12 136.24) (width 0.25) (layer "F.Cu") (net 3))
 (segment (start 147.16 72) (end 150.19 75.03) (width 0.25) (layer "F.Cu") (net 3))
 (segment (start 134.8 72) (end 147.16 72) (width 0.25) (layer "F.Cu") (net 3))
 (via (at 149.83846 143.5) (size 0.8) (drill 0.4) (layers "F.Cu" "B.Cu") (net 3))
 (segment (start 149.31 77.96) (end 149.31 76.43) (width 0.25) (layer "F.Cu") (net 1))
 (segment (start 154.16 135.78) (end 154.16 82.81) (width 0.25) (layer "F.Cu") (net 1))
 (segment (start 147.430768 143.5) (end 147.430768 142.509232) (width 0.25) (layer "F.Cu") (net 1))
 (segment (start 146.88 74) (end 134.8 74) (width 0.25) (layer "F.Cu") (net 1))
 (segment (start 149.31 76.43) (end 146.88 74) (width 0.25) (layer "F.Cu") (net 1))
 (segment (start 154.16 82.81) (end 149.31 77.96) (width 0.25) (layer "F.Cu") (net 1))
 (segment (start 147.430768 142.509232) (end 154.16 135.78) (width 0.25) (layer "F.Cu") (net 1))
 (via (at 147.430768 143.5) (size 0.8) (drill 0.4) (layers "F.Cu" "B.Cu") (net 1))
 (segment (start 145.11 143.5) (end 153.16 135.45) (width 0.25) (layer "F.Cu") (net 2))
 (segment (start 153.16 135.45) (end 153.16 82.55) (width 0.25) (layer "F.Cu") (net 2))
 (segment (start 145.023076 143.5) (end 145.11 143.5) (width 0.25) (layer "F.Cu") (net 2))
 (segment (start 153.16 82.55) (end 146.61 76) (width 0.25) (layer "F.Cu") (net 2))
 (segment (start 146.61 76) (end 134.8 76) (width 0.25) (layer "F.Cu") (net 2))
 (via (at 145.023076 143.5) (size 0.8) (drill 0.4) (layers "F.Cu" "B.Cu") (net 2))
 (segment (start 152.13 135.38) (end 152.13 82.27) (width 0.25) (layer "F.Cu") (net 9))
 (segment (start 147.86 78) (end 134.8 78) (width 0.25) (layer "F.Cu") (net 9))
 (segment (start 149.53 137.98) (end 152.13 135.38) (width 0.25) (layer "F.Cu") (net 9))
 (segment (start 142.615384 141.074616) (end 145.71 137.98) (width 0.25) (layer "F.Cu") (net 9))
 (segment (start 145.71 137.98) (end 149.53 137.98) (width 0.25) (layer "F.Cu") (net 9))
 (segment (start 152.13 82.27) (end 147.86 78) (width 0.25) (layer "F.Cu") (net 9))
 (segment (start 142.615384 143.5) (end 142.615384 141.074616) (width 0.25) (layer "F.Cu") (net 9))
 (via (at 142.615384 143.5) (size 0.8) (drill 0.4) (layers "F.Cu" "B.Cu") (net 9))
 (segment (start 140.207692 143.5) (end 140.207692 138.422308) (width 0.25) (layer "F.Cu") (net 6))
 (segment (start 141.64 136.99) (end 149.58 136.99) (width 0.25) (layer "F.Cu") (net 6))
 (segment (start 151.08 82.053838) (end 149.026162 80) (width 0.25) (layer "F.Cu") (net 6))
 (segment (start 149.58 136.99) (end 151.08 135.49) (width 0.25) (layer "F.Cu") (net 6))
 (segment (start 151.08 135.49) (end 151.08 82.053838) (width 0.25) (layer "F.Cu") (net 6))
 (segment (start 140.207692 138.422308) (end 141.64 136.99) (width 0.25) (layer "F.Cu") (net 6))
 (segment (start 149.026162 80) (end 134.8 80) (width 0.25) (layer "F.Cu") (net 6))
 (via (at 140.207692 143.5) (size 0.8) (drill 0.4) (layers "F.Cu" "B.Cu") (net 6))
 (segment (start 130.6 74.8) (end 146 74.8) (width 0.25) (layer "B.Cu") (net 12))
 (segment (start 146 74.8) (end 154.13 82.93) (width 0.25) (layer "B.Cu") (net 12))
 (segment (start 161.87692 140.53692) (end 161.87692 143.5) (width 0.25) (layer "B.Cu") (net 12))
 (segment (start 127.8 72) (end 130.6 74.8) (width 0.25) (layer "B.Cu") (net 12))
 (segment (start 157.07 138.48) (end 159.82 138.48) (width 0.25) (layer "B.Cu") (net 12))
 (segment (start 159.82 138.48) (end 161.87692 140.53692) (width 0.25) (layer "B.Cu") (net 12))
 (segment (start 154.13 82.93) (end 154.13 135.54) (width 0.25) (layer "B.Cu") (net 12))
 (segment (start 154.13 135.54) (end 157.07 138.48) (width 0.25) (layer "B.Cu") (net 12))
 (segment (start 154.653844 140.403844) (end 151.23 136.98) (width 0.25) (layer "B.Cu") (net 16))
 (segment (start 154.653844 143.5) (end 154.653844 140.403844) (width 0.25) (layer "B.Cu") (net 16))
 (segment (start 151.23 136.98) (end 151.23 82.203838) (width 0.25) (layer "B.Cu") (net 16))
 (segment (start 151.23 82.203838) (end 149.726162 80.7) (width 0.25) (layer "B.Cu") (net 16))
 (segment (start 130.5 80.7) (end 127.8 78) (width 0.25) (layer "B.Cu") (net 16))
 (segment (start 149.726162 80.7) (end 130.5 80.7) (width 0.25) (layer "B.Cu") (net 16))
 (segment (start 150.1 76.39) (end 154.86 76.39) (width 0.25) (layer "B.Cu") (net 15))
 (segment (start 154.86 76.39) (end 156.025 77.555) (width 0.25) (layer "B.Cu") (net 15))
 (segment (start 145.71 72) (end 150.1 76.39) (width 0.25) (layer "B.Cu") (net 15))
 (segment (start 166.692304 138.502304) (end 166.692304 143.57) (width 0.25) (layer "B.Cu") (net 15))
 (segment (start 157.193838 136.62) (end 164.81 136.62) (width 0.25) (layer "B.Cu") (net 15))
 (segment (start 156.025 77.555) (end 156.025 135.451162) (width 0.25) (layer "B.Cu") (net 15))
 (segment (start 156.025 135.451162) (end 157.193838 136.62) (width 0.25) (layer "B.Cu") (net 15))
 (segment (start 141.8 72) (end 145.71 72) (width 0.25) (layer "B.Cu") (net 15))
 (segment (start 164.81 136.62) (end 166.692304 138.502304) (width 0.25) (layer "B.Cu") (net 15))
 (segment (start 156.85 139.66) (end 153.09 135.9) (width 0.25) (layer "B.Cu") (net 11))
 (segment (start 148.376396 78) (end 141.8 78) (width 0.25) (layer "B.Cu") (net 11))
 (segment (start 153.09 82.713604) (end 148.376396 78) (width 0.25) (layer "B.Cu") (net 11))
 (segment (start 159.469228 140.849228) (end 158.28 139.66) (width 0.25) (layer "B.Cu") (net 11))
 (segment (start 159.469228 143.5) (end 159.469228 140.849228) (width 0.25) (layer "B.Cu") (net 11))
 (segment (start 153.09 135.9) (end 153.09 82.713604) (width 0.25) (layer "B.Cu") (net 11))
 (segment (start 158.28 139.66) (end 156.85 139.66) (width 0.25) (layer "B.Cu") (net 11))
 (segment (start 161.75 137.65) (end 157.3 137.65) (width 0.25) (layer "B.Cu") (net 13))
 (segment (start 146.06 74.07) (end 136.87 74.07) (width 0.25) (layer "B.Cu") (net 13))
 (segment (start 157.3 137.65) (end 155.1 135.45) (width 0.25) (layer "B.Cu") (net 13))
 (segment (start 155.1 135.45) (end 155.1 83.11) (width 0.25) (layer "B.Cu") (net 13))
 (segment (start 164.284612 140.184612) (end 161.75 137.65) (width 0.25) (layer "B.Cu") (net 13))
 (segment (start 164.284612 143.5) (end 164.284612 140.184612) (width 0.25) (layer "B.Cu") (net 13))
 (segment (start 155.1 83.11) (end 146.06 74.07) (width 0.25) (layer "B.Cu") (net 13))
 (segment (start 136.87 74.07) (end 134.8 72) (width 0.25) (layer "B.Cu") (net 13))
 (segment (start 149.62 79.88) (end 152.08 82.34) (width 0.25) (layer "B.Cu") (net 14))
 (segment (start 152.08 82.34) (end 152.08 136.41) (width 0.25) (layer "B.Cu") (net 14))
 (segment (start 134.8 78) (end 136.68 79.88) (width 0.25) (layer "B.Cu") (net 14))
 (segment (start 152.08 136.41) (end 157.061536 141.391536) (width 0.25) (layer "B.Cu") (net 14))
 (segment (start 136.68 79.88) (end 149.62 79.88) (width 0.25) (layer "B.Cu") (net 14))
 (segment (start 157.061536 141.391536) (end 157.061536 143.5) (width 0.25) (layer "B.Cu") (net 14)))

